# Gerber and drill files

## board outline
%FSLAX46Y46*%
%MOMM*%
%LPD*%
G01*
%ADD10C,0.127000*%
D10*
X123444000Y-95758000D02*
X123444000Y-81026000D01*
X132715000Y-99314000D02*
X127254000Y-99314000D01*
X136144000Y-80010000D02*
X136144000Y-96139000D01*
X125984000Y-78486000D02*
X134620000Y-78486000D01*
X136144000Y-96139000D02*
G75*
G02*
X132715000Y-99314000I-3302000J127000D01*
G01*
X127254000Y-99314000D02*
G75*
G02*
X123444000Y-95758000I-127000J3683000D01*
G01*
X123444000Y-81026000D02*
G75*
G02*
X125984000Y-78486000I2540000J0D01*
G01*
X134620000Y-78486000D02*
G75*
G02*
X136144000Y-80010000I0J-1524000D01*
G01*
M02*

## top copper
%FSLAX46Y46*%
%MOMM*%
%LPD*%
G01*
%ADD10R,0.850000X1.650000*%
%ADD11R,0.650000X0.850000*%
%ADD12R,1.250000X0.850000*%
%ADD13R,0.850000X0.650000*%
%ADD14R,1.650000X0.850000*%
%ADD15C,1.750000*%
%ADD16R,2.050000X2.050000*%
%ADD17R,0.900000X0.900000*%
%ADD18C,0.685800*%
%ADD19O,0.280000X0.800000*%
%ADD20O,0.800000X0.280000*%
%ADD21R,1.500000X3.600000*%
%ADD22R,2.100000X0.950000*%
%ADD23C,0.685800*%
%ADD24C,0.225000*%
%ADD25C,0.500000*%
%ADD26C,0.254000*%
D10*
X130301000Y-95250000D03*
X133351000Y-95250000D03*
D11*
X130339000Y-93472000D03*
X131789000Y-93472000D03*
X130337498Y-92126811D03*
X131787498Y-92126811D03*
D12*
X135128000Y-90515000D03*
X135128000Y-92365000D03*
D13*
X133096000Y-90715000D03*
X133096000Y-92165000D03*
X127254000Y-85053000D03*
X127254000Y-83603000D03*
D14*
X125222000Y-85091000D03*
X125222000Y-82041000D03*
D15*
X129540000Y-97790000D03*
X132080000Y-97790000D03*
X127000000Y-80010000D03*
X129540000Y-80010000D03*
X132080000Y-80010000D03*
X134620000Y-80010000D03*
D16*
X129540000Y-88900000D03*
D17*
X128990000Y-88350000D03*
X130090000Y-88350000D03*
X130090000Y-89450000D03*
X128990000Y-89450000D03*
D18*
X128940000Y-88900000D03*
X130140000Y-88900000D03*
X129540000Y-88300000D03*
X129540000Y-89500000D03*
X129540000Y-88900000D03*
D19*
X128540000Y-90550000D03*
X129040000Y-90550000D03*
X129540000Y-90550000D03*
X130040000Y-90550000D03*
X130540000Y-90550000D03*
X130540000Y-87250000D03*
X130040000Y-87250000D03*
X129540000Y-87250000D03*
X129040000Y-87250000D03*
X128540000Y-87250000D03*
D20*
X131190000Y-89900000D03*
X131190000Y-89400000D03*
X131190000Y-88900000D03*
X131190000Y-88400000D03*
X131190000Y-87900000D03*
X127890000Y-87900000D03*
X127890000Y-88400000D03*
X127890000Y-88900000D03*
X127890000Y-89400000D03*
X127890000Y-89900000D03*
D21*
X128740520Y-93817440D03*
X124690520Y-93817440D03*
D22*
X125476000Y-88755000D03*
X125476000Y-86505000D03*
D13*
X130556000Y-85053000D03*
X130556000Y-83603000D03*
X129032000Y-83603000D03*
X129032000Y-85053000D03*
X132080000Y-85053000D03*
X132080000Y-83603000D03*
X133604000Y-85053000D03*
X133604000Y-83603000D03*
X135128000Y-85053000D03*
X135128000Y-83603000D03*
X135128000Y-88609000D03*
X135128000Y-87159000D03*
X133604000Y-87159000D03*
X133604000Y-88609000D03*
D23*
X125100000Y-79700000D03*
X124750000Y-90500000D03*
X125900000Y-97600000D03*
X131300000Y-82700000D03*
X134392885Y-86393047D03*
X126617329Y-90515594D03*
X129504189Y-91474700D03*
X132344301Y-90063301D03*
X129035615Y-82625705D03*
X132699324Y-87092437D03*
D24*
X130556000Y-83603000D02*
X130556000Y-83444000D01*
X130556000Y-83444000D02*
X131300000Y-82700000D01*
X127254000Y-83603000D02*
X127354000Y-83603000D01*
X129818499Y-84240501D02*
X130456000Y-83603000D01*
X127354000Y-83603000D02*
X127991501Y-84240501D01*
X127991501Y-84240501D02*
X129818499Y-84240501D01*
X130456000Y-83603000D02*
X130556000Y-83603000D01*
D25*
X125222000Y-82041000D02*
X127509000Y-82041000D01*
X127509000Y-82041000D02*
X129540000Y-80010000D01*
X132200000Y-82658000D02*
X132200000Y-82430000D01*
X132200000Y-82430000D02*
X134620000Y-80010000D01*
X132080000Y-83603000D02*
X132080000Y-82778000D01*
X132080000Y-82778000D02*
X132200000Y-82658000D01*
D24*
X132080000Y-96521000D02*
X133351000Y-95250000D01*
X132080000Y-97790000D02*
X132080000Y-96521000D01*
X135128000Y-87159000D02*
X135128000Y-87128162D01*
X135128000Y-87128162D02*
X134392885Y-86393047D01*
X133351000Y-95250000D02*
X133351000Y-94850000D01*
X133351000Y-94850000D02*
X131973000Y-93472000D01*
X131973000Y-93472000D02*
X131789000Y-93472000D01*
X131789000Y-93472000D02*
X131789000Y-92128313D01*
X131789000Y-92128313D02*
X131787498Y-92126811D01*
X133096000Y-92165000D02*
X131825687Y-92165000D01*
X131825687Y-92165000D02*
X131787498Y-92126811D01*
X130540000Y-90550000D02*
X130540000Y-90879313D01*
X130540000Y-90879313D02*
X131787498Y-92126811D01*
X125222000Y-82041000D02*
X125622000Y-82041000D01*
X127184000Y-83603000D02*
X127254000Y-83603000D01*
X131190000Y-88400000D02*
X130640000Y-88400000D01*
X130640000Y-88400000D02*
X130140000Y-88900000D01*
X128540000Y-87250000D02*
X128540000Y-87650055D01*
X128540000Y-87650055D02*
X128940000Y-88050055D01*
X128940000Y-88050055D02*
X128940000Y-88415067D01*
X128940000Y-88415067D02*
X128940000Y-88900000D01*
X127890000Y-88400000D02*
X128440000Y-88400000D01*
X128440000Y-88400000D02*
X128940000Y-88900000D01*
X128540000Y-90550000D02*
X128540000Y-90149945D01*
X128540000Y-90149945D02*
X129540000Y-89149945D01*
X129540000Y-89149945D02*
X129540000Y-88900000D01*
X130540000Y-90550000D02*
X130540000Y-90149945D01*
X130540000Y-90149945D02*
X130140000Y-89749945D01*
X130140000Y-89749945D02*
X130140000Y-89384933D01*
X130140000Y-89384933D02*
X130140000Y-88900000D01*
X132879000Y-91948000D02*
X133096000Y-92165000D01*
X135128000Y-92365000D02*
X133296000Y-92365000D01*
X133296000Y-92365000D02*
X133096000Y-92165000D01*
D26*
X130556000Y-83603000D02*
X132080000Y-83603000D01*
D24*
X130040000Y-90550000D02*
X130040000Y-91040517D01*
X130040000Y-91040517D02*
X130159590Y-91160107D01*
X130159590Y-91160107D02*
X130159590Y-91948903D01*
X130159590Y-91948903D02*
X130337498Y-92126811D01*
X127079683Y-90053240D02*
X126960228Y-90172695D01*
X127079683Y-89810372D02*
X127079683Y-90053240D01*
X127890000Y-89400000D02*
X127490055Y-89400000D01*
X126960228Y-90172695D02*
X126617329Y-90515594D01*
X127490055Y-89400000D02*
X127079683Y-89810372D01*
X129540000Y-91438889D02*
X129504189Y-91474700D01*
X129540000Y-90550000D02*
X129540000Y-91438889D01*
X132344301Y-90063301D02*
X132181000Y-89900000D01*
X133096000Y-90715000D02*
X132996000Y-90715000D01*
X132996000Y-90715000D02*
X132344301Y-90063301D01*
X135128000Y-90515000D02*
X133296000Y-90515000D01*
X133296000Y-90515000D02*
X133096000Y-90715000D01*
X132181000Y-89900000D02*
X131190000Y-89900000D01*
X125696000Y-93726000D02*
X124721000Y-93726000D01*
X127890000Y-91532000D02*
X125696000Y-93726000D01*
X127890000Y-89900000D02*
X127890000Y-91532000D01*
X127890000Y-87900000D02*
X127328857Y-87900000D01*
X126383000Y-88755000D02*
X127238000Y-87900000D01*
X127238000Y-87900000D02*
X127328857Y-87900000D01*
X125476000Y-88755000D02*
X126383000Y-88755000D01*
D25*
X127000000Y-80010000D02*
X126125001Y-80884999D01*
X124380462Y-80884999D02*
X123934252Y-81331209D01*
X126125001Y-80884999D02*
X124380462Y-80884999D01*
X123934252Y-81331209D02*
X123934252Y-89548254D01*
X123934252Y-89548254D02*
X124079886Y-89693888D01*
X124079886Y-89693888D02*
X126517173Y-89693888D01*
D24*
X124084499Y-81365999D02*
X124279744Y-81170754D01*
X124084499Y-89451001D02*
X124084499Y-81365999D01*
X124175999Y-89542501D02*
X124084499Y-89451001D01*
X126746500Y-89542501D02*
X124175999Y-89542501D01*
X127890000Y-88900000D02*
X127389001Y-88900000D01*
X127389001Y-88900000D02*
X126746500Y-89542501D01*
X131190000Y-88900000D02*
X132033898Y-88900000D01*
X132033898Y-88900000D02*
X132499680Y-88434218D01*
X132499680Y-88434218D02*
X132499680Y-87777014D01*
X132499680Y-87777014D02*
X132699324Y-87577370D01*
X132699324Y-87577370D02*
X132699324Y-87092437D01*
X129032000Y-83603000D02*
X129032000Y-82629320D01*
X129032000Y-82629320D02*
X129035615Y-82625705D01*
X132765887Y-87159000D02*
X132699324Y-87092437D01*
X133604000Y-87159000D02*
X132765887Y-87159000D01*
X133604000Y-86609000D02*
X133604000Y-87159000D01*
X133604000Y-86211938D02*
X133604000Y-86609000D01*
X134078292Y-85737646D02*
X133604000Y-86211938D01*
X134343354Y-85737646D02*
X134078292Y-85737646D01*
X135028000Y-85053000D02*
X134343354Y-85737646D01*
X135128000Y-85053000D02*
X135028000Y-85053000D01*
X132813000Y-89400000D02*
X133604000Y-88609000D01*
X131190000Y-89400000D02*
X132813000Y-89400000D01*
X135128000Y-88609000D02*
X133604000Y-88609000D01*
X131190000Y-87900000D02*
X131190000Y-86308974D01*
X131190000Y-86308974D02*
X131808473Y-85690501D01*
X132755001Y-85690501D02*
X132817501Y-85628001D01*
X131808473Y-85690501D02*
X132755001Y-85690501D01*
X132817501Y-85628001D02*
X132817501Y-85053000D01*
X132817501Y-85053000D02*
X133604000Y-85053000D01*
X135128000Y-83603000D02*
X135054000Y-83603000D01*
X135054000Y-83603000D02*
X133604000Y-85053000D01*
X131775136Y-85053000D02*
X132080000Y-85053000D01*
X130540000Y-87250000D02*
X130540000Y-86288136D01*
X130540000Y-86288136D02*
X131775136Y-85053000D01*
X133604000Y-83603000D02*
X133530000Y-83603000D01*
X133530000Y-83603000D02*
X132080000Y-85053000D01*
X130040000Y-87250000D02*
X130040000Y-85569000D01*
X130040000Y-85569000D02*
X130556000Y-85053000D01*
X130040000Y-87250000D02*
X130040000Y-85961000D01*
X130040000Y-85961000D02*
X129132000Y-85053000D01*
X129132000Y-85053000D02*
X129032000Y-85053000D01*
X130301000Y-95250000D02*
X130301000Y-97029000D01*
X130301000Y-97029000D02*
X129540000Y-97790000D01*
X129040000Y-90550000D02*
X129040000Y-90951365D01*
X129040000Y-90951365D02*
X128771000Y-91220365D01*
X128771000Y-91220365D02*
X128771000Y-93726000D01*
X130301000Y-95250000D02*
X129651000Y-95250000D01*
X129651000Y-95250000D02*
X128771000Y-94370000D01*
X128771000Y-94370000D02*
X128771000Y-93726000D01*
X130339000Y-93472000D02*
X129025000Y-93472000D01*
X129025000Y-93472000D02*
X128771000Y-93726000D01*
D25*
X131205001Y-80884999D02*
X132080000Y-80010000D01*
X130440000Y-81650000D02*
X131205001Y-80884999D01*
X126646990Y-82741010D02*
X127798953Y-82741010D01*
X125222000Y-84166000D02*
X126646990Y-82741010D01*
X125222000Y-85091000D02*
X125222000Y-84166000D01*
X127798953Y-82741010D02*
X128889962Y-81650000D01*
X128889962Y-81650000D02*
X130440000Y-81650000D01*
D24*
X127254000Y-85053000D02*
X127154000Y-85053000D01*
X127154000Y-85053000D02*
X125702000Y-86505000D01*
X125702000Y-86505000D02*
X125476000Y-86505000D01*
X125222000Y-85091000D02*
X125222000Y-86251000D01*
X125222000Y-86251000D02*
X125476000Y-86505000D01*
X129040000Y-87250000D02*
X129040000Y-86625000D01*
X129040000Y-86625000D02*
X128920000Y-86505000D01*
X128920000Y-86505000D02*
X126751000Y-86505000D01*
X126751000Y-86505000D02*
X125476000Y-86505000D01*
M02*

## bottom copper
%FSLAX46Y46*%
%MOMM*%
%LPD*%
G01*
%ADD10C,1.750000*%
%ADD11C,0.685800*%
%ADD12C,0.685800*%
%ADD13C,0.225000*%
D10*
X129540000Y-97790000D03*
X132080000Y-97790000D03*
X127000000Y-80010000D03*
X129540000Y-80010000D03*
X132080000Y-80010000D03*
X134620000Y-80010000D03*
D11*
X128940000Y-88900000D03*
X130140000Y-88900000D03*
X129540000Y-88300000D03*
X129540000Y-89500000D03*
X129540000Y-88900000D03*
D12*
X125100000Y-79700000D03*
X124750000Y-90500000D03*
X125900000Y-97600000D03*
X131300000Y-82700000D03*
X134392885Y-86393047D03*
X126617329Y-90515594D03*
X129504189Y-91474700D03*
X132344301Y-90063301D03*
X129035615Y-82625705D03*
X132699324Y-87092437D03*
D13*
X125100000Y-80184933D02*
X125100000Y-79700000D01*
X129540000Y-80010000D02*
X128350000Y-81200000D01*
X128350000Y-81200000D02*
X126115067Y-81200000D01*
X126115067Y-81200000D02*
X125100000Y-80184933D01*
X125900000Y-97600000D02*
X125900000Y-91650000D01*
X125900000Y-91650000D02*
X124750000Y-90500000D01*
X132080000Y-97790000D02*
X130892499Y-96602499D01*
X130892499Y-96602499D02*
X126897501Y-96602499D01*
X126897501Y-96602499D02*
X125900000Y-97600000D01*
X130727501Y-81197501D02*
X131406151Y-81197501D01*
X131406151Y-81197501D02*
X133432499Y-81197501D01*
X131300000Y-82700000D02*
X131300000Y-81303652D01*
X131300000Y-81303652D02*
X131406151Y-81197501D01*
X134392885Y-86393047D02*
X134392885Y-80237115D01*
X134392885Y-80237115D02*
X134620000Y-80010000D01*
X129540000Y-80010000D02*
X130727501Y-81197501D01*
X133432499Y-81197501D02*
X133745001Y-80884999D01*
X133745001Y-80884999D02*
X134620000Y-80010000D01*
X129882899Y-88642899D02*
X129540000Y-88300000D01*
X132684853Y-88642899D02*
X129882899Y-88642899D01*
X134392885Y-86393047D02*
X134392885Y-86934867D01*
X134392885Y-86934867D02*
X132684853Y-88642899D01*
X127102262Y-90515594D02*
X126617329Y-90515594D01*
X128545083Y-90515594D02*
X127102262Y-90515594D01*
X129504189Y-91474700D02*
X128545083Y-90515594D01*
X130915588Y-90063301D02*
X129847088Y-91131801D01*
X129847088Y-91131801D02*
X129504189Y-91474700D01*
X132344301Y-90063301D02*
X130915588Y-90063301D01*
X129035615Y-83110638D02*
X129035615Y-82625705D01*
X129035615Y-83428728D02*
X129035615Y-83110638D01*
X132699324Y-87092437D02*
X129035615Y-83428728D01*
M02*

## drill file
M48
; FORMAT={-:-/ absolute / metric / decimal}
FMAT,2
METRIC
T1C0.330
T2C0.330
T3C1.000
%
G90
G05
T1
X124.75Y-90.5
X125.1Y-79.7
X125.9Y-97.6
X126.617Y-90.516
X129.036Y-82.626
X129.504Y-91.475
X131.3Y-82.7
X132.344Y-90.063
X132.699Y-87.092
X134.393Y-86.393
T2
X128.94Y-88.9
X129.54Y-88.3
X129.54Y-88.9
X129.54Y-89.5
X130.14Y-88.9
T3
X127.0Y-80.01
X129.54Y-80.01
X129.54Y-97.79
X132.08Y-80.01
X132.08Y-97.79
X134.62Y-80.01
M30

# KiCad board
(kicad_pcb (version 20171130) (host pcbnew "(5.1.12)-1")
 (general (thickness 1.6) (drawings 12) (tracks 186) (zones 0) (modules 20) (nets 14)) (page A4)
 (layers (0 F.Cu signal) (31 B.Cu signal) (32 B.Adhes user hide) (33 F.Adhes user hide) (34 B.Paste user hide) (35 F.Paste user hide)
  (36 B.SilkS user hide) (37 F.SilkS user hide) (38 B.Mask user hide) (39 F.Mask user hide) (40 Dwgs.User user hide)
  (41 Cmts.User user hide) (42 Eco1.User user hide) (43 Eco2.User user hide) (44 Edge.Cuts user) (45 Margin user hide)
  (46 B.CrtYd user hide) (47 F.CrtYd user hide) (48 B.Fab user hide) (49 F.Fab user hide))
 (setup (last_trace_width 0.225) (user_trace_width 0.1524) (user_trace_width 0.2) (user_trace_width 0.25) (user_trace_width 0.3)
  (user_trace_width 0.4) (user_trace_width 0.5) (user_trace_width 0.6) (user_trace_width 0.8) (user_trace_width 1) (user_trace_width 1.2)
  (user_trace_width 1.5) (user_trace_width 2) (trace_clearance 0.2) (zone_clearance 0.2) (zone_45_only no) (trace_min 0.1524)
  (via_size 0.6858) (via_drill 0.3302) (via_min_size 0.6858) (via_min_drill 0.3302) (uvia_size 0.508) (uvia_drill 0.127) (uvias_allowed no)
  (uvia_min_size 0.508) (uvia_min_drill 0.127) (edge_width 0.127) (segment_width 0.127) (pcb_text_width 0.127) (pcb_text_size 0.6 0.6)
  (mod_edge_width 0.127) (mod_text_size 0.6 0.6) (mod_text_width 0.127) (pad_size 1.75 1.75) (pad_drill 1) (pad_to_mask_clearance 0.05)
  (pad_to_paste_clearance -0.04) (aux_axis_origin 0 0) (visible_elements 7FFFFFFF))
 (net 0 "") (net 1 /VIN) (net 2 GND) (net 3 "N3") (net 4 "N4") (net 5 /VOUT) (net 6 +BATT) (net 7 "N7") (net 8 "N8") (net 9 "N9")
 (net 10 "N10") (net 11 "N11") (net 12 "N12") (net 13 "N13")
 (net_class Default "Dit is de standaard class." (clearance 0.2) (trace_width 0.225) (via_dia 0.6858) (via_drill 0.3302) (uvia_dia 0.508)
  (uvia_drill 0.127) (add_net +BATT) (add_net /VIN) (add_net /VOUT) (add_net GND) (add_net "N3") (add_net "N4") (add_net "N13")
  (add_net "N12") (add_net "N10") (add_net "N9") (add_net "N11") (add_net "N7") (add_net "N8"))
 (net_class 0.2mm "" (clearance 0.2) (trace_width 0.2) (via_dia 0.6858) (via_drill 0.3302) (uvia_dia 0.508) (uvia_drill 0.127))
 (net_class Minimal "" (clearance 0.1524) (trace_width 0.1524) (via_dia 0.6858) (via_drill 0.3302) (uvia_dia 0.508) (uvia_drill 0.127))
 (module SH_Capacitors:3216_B (layer F.Cu) (at 131.826 95.25) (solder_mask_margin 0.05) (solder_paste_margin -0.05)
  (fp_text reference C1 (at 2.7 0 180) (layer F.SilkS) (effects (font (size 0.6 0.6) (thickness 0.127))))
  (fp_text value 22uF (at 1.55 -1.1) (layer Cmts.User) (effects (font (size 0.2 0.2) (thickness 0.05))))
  (pad 1 smd rect (at -1.525 0) (size 0.85 1.65) (layers F.Cu F.Paste F.Mask) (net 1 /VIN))
  (pad 2 smd rect (at 1.525 0) (size 0.85 1.65) (layers F.Cu F.Paste F.Mask) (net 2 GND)))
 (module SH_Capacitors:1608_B (layer F.Cu) (at 131.064 93.472) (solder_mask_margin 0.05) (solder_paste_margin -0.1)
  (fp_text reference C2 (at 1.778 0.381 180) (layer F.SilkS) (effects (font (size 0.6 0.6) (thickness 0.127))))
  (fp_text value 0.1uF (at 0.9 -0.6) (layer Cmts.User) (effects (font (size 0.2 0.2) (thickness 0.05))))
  (pad 1 smd rect (at -0.725 0) (size 0.65 0.85) (layers F.Cu F.Paste F.Mask) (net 1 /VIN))
  (pad 2 smd rect (at 0.725 0) (size 0.65 0.85) (layers F.Cu F.Paste F.Mask) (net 2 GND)))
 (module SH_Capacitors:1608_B (layer F.Cu) (at 131.062498 92.126811) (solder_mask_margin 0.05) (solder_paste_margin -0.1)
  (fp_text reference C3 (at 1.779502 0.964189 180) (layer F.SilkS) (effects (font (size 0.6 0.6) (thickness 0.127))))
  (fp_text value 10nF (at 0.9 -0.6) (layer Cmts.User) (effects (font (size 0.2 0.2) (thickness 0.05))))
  (pad 1 smd rect (at -0.725 0) (size 0.65 0.85) (layers F.Cu F.Paste F.Mask) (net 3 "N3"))
  (pad 2 smd rect (at 0.725 0) (size 0.65 0.85) (layers F.Cu F.Paste F.Mask) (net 2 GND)))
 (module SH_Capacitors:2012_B (layer F.Cu) (at 135.128 91.44 270) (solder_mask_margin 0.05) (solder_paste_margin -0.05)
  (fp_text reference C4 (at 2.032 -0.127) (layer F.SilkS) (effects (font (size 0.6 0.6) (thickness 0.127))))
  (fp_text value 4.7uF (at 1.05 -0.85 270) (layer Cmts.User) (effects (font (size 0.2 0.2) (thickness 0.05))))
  (pad 1 smd rect (at -0.925 0 270) (size 0.85 1.25) (layers F.Cu F.Paste F.Mask) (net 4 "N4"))
  (pad 2 smd rect (at 0.925 0 270) (size 0.85 1.25) (layers F.Cu F.Paste F.Mask) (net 2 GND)))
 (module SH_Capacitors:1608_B (layer F.Cu) (at 133.096 91.44 270) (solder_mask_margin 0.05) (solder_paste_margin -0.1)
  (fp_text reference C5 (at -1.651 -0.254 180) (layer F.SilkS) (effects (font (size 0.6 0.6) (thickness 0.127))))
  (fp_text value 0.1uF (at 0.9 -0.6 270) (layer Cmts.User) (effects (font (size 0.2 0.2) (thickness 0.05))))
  (pad 1 smd rect (at -0.725 0 270) (size 0.65 0.85) (layers F.Cu F.Paste F.Mask) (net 4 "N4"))
  (pad 2 smd rect (at 0.725 0 270) (size 0.65 0.85) (layers F.Cu F.Paste F.Mask) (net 2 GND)))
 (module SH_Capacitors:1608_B (layer F.Cu) (at 127.254 84.328 90) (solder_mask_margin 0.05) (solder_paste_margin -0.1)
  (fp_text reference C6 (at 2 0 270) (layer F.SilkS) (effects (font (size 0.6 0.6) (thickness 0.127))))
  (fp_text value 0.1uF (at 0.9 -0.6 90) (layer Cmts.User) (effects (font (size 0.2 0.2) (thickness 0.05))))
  (pad 1 smd rect (at -0.725 0 90) (size 0.65 0.85) (layers F.Cu F.Paste F.Mask) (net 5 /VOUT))
  (pad 2 smd rect (at 0.725 0 90) (size 0.65 0.85) (layers F.Cu F.Paste F.Mask) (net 2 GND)))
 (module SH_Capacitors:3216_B (layer F.Cu) (at 125.222 83.566 90) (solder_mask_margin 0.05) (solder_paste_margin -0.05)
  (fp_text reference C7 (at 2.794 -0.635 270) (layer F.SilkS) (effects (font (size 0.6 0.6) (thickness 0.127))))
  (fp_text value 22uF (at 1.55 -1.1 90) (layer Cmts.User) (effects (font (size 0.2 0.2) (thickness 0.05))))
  (pad 1 smd rect (at -1.525 0 90) (size 0.85 1.65) (layers F.Cu F.Paste F.Mask) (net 5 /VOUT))
  (pad 2 smd rect (at 1.525 0 90) (size 0.85 1.65) (layers F.Cu F.Paste F.Mask) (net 2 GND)))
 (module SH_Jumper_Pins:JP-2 (layer F.Cu) (at 130.81 97.79)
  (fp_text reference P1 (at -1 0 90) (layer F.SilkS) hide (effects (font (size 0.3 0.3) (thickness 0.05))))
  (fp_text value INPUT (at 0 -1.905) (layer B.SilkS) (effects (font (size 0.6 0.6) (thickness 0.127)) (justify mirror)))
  (pad 1 thru_hole circle (at -1.27 0) (size 1.75 1.75) (drill 1) (layers *.Cu *.Mask) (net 1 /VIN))
  (pad 2 thru_hole circle (at 1.27 0) (size 1.75 1.75) (drill 1) (layers *.Cu *.Mask) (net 2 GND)))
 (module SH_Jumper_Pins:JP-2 (layer F.Cu) (at 128.27 80.01)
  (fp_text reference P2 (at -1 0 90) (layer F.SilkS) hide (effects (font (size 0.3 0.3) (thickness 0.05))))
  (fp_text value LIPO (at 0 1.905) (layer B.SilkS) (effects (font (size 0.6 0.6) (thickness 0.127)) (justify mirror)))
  (pad 1 thru_hole circle (at -1.27 0) (size 1.75 1.75) (drill 1) (layers *.Cu *.Mask) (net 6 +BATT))
  (pad 2 thru_hole circle (at 1.27 0) (size 1.75 1.75) (drill 1) (layers *.Cu *.Mask) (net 2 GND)))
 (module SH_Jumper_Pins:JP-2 (layer F.Cu) (at 133.35 80.01)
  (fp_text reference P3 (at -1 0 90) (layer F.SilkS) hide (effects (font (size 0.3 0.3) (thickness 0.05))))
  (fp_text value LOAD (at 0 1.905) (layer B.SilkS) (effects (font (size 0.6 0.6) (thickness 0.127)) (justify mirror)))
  (pad 1 thru_hole circle (at -1.27 0) (size 1.75 1.75) (drill 1) (layers *.Cu *.Mask) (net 5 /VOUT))
  (pad 2 thru_hole circle (at 1.27 0) (size 1.75 1.75) (drill 1) (layers *.Cu *.Mask) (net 2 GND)))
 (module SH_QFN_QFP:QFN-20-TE (layer F.Cu) (at 129.54 88.9) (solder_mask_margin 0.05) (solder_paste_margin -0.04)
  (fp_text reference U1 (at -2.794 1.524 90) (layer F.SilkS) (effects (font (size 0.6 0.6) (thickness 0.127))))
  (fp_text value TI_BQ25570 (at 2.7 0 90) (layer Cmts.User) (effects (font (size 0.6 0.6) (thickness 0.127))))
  (pad 21 smd rect (at 0 0) (size 2.05 2.05) (layers F.Cu F.Mask) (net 2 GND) (zone_connect 2))
  (pad 21 smd rect (at -0.55 -0.55) (size 0.9 0.9) (layers F.Cu F.Paste F.Mask) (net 2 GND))
  (pad 21 smd rect (at 0.55 -0.55) (size 0.9 0.9) (layers F.Cu F.Paste F.Mask) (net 2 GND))
  (pad 21 smd rect (at 0.55 0.55) (size 0.9 0.9) (layers F.Cu F.Paste F.Mask) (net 2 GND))
  (pad 21 smd rect (at -0.55 0.55) (size 0.9 0.9) (layers F.Cu F.Paste F.Mask) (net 2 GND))
  (pad 21 thru_hole circle (at -0.6 0) (size 0.6858 0.6858) (drill 0.3302) (layers *.Cu) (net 2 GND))
  (pad 21 thru_hole circle (at 0.6 0) (size 0.6858 0.6858) (drill 0.3302) (layers *.Cu) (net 2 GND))
  (pad 21 thru_hole circle (at 0 -0.6) (size 0.6858 0.6858) (drill 0.3302) (layers *.Cu) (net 2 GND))
  (pad 21 thru_hole circle (at 0 0.6) (size 0.6858 0.6858) (drill 0.3302) (layers *.Cu) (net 2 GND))
  (pad 21 thru_hole circle (at 0 0) (size 0.6858 0.6858) (drill 0.3302) (layers *.Cu) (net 2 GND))
  (pad 1 smd oval (at -1 1.65) (size 0.28 0.8) (layers F.Cu F.Paste F.Mask) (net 2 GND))
  (pad 2 smd oval (at -0.5 1.65) (size 0.28 0.8) (layers F.Cu F.Paste F.Mask) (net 1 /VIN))
  (pad 3 smd oval (at 0 1.65) (size 0.28 0.8) (layers F.Cu F.Paste F.Mask) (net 4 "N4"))
  (pad 4 smd oval (at 0.5 1.65) (size 0.28 0.8) (layers F.Cu F.Paste F.Mask) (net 3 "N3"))
  (pad 5 smd oval (at 1 1.65) (size 0.28 0.8) (layers F.Cu F.Paste F.Mask) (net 2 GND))
  (pad 11 smd oval (at 1 -1.65) (size 0.28 0.8) (layers F.Cu F.Paste F.Mask) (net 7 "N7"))
  (pad 12 smd oval (at 0.5 -1.65) (size 0.28 0.8) (layers F.Cu F.Paste F.Mask) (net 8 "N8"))
  (pad 13 smd oval (at 0 -1.65) (size 0.28 0.8) (layers F.Cu F.Paste F.Mask))
  (pad 14 smd oval (at -0.5 -1.65) (size 0.28 0.8) (layers F.Cu F.Paste F.Mask) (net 5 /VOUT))
  (pad 15 smd oval (at -1 -1.65) (size 0.28 0.8) (layers F.Cu F.Paste F.Mask) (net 2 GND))
  (pad 6 smd oval (at 1.65 1 90) (size 0.28 0.8) (layers F.Cu F.Paste F.Mask) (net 4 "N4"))
  (pad 7 smd oval (at 1.65 0.5 90) (size 0.28 0.8) (layers F.Cu F.Paste F.Mask) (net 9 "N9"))
  (pad 8 smd oval (at 1.65 0 90) (size 0.28 0.8) (layers F.Cu F.Paste F.Mask) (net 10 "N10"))
  (pad 9 smd oval (at 1.65 -0.5 90) (size 0.28 0.8) (layers F.Cu F.Paste F.Mask) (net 2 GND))
  (pad 10 smd oval (at 1.65 -1 90) (size 0.28 0.8) (layers F.Cu F.Paste F.Mask) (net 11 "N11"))
  (pad 16 smd oval (at -1.65 -1 90) (size 0.28 0.8) (layers F.Cu F.Paste F.Mask) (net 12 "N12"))
  (pad 17 smd oval (at -1.65 -0.5 90) (size 0.28 0.8) (layers F.Cu F.Paste F.Mask) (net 2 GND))
  (pad 18 smd oval (at -1.65 0 90) (size 0.28 0.8) (layers F.Cu F.Paste F.Mask) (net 6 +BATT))
  (pad 19 smd oval (at -1.65 0.5 90) (size 0.28 0.8) (layers F.Cu F.Paste F.Mask) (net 4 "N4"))
  (pad 20 smd oval (at -1.65 1 90) (size 0.28 0.8) (layers F.Cu F.Paste F.Mask) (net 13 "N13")))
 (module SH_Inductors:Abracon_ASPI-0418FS (layer F.Cu) (at 126.71552 93.81744 180) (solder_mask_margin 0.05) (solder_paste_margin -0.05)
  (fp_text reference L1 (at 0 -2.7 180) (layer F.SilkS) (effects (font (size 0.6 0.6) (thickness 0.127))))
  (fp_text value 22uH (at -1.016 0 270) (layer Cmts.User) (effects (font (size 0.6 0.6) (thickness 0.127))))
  (pad 1 smd rect (at -2.025 0 180) (size 1.5 3.6) (layers F.Cu F.Paste F.Mask) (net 1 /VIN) (zone_connect 2))
  (pad 2 smd rect (at 2.025 0 180) (size 1.5 3.6) (layers F.Cu F.Paste F.Mask) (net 13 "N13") (zone_connect 2)))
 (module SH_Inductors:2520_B (layer F.Cu) (at 125.476 87.63 90) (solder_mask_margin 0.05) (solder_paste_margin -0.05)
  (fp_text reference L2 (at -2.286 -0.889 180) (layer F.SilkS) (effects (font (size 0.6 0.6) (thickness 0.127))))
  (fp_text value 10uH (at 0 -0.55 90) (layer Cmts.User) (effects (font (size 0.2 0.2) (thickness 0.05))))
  (pad 1 smd rect (at -1.125 0 90) (size 0.95 2.1) (layers F.Cu F.Paste F.Mask) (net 12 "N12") (zone_connect 2))
  (pad 2 smd rect (at 1.125 0 90) (size 0.95 2.1) (layers F.Cu F.Paste F.Mask) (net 5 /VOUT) (zone_connect 2)))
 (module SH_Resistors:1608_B (layer F.Cu) (at 130.556 84.328 90) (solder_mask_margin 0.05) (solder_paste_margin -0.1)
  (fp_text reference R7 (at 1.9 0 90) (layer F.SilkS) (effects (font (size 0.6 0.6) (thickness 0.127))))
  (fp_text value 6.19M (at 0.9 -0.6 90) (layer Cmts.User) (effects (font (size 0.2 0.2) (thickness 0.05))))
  (pad 1 smd rect (at -0.725 0 90) (size 0.65 0.85) (layers F.Cu F.Paste F.Mask) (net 8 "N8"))
  (pad 2 smd rect (at 0.725 0 90) (size 0.65 0.85) (layers F.Cu F.Paste F.Mask) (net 2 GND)))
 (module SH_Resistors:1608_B (layer F.Cu) (at 129.032 84.328 270) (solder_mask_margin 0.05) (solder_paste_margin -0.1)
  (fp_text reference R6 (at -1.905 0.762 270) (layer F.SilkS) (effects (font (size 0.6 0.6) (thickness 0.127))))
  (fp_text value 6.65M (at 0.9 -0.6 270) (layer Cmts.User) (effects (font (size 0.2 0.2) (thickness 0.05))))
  (pad 1 smd rect (at -0.725 0 270) (size 0.65 0.85) (layers F.Cu F.Paste F.Mask) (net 10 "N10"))
  (pad 2 smd rect (at 0.725 0 270) (size 0.65 0.85) (layers F.Cu F.Paste F.Mask) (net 8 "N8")))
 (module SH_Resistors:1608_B (layer F.Cu) (at 132.08 84.328 90) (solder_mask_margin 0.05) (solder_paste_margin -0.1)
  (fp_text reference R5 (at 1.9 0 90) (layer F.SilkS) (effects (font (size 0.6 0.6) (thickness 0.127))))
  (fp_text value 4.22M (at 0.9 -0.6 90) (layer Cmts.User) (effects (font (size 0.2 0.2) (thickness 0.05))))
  (pad 1 smd rect (at -0.725 0 90) (size 0.65 0.85) (layers F.Cu F.Paste F.Mask) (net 7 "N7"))
  (pad 2 smd rect (at 0.725 0 90) (size 0.65 0.85) (layers F.Cu F.Paste F.Mask) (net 2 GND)))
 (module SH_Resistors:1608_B (layer F.Cu) (at 133.604 84.328 90) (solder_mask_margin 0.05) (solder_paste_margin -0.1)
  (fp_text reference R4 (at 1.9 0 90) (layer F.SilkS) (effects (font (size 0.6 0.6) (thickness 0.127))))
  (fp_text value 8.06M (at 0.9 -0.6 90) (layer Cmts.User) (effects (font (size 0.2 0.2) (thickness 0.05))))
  (pad 1 smd rect (at -0.725 0 90) (size 0.65 0.85) (layers F.Cu F.Paste F.Mask) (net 11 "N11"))
  (pad 2 smd rect (at 0.725 0 90) (size 0.65 0.85) (layers F.Cu F.Paste F.Mask) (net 7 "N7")))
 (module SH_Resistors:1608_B (layer F.Cu) (at 135.128 84.328 90) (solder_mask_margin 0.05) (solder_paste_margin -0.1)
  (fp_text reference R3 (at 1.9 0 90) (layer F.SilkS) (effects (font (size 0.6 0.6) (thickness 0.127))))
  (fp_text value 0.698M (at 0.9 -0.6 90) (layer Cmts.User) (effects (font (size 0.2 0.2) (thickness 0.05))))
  (pad 1 smd rect (at -0.725 0 90) (size 0.65 0.85) (layers F.Cu F.Paste F.Mask) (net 10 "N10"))
  (pad 2 smd rect (at 0.725 0 90) (size 0.65 0.85) (layers F.Cu F.Paste F.Mask) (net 11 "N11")))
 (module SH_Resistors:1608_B (layer F.Cu) (at 135.128 87.884 90) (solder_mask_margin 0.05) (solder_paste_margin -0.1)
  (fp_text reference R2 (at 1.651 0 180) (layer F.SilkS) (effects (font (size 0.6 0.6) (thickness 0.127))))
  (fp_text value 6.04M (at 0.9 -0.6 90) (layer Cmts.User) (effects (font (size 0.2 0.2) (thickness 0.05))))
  (pad 1 smd rect (at -0.725 0 90) (size 0.65 0.85) (layers F.Cu F.Paste F.Mask) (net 9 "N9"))
  (pad 2 smd rect (at 0.725 0 90) (size 0.65 0.85) (layers F.Cu F.Paste F.Mask) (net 2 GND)))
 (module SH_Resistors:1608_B (layer F.Cu) (at 133.604 87.884 270) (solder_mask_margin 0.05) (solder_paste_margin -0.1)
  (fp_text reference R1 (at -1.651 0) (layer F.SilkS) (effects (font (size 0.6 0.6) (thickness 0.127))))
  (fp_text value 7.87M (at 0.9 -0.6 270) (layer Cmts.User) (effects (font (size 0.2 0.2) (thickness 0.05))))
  (pad 1 smd rect (at -0.725 0 270) (size 0.65 0.85) (layers F.Cu F.Paste F.Mask) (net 10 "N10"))
  (pad 2 smd rect (at 0.725 0 270) (size 0.65 0.85) (layers F.Cu F.Paste F.Mask) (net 9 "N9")))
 (gr_line (start 123.444 95.758) (end 123.444 81.026) (angle 90) (layer Edge.Cuts) (width 0.127))
 (gr_line (start 132.715 99.314) (end 127.254 99.314) (angle 90) (layer Edge.Cuts) (width 0.127))
 (gr_line (start 136.144 80.01) (end 136.144 96.139) (angle 90) (layer Edge.Cuts) (width 0.127))
 (gr_line (start 125.984 78.486) (end 134.62 78.486) (angle 90) (layer Edge.Cuts) (width 0.127))
 (gr_arc (start 132.842 96.012) (end 136.144 96.139) (angle 90) (layer Edge.Cuts) (width 0.127))
 (gr_arc (start 127.127 95.631) (end 127.254 99.314) (angle 90) (layer Edge.Cuts) (width 0.127))
 (gr_arc (start 125.984 81.026) (end 123.444 81.026) (angle 90) (layer Edge.Cuts) (width 0.127))
 (gr_arc (start 134.62 80.01) (end 134.62 78.486) (angle 90) (layer Edge.Cuts) (width 0.127))
 (segment (start 125.1 80.184933) (end 125.1 79.7) (width 0.225) (layer B.Cu) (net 2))
 (segment (start 129.54 80.01) (end 128.35 81.2) (width 0.225) (layer B.Cu) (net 2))
 (segment (start 128.35 81.2) (end 126.115067 81.2) (width 0.225) (layer B.Cu) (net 2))
 (segment (start 126.115067 81.2) (end 125.1 80.184933) (width 0.225) (layer B.Cu) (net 2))
 (segment (start 125.9 97.6) (end 125.9 91.65) (width 0.225) (layer B.Cu) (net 2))
 (segment (start 125.9 91.65) (end 124.75 90.5) (width 0.225) (layer B.Cu) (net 2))
 (segment (start 132.08 97.79) (end 130.892499 96.602499) (width 0.225) (layer B.Cu) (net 2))
 (segment (start 130.892499 96.602499) (end 126.897501 96.602499) (width 0.225) (layer B.Cu) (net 2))
 (segment (start 126.897501 96.602499) (end 125.9 97.6) (width 0.225) (layer B.Cu) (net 2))
 (segment (start 130.727501 81.197501) (end 131.406151 81.197501) (width 0.225) (layer B.Cu) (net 2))
 (segment (start 131.406151 81.197501) (end 133.432499 81.197501) (width 0.225) (layer B.Cu) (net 2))
 (segment (start 131.3 82.7) (end 131.3 81.303652) (width 0.225) (layer B.Cu) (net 2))
 (segment (start 131.3 81.303652) (end 131.406151 81.197501) (width 0.225) (layer B.Cu) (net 2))
 (segment (start 130.556 83.603) (end 130.556 83.444) (width 0.225) (layer F.Cu) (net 2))
 (segment (start 130.556 83.444) (end 131.3 82.7) (width 0.225) (layer F.Cu) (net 2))
 (segment (start 134.392885 86.393047) (end 134.392885 80.237115) (width 0.225) (layer B.Cu) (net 2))
 (segment (start 134.392885 80.237115) (end 134.62 80.01) (width 0.225) (layer B.Cu) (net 2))
 (segment (start 129.54 80.01) (end 130.727501 81.197501) (width 0.225) (layer B.Cu) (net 2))
 (segment (start 133.432499 81.197501) (end 133.745001 80.884999) (width 0.225) (layer B.Cu) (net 2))
 (segment (start 133.745001 80.884999) (end 134.62 80.01) (width 0.225) (layer B.Cu) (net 2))
 (segment (start 127.254 83.603) (end 127.354 83.603) (width 0.225) (layer F.Cu) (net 2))
 (segment (start 129.818499 84.240501) (end 130.456 83.603) (width 0.225) (layer F.Cu) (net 2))
 (segment (start 127.354 83.603) (end 127.991501 84.240501) (width 0.225) (layer F.Cu) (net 2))
 (segment (start 127.991501 84.240501) (end 129.818499 84.240501) (width 0.225) (layer F.Cu) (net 2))
 (segment (start 130.456 83.603) (end 130.556 83.603) (width 0.225) (layer F.Cu) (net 2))
 (segment (start 125.222 82.041) (end 127.509 82.041) (width 0.5) (layer F.Cu) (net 2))
 (segment (start 127.509 82.041) (end 129.54 80.01) (width 0.5) (layer F.Cu) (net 2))
 (segment (start 132.2 82.658) (end 132.2 82.43) (width 0.5) (layer F.Cu) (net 2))
 (segment (start 132.2 82.43) (end 134.62 80.01) (width 0.5) (layer F.Cu) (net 2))
 (segment (start 132.08 83.603) (end 132.08 82.778) (width 0.5) (layer F.Cu) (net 2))
 (segment (start 132.08 82.778) (end 132.2 82.658) (width 0.5) (layer F.Cu) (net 2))
 (segment (start 132.08 96.521) (end 133.351 95.25) (width 0.225) (layer F.Cu) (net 2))
 (segment (start 132.08 97.79) (end 132.08 96.521) (width 0.225) (layer F.Cu) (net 2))
 (segment (start 129.882899 88.642899) (end 129.54 88.3) (width 0.225) (layer B.Cu) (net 2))
 (segment (start 132.684853 88.642899) (end 129.882899 88.642899) (width 0.225) (layer B.Cu) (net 2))
 (segment (start 134.392885 86.393047) (end 134.392885 86.934867) (width 0.225) (layer B.Cu) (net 2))
 (segment (start 134.392885 86.934867) (end 132.684853 88.642899) (width 0.225) (layer B.Cu) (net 2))
 (segment (start 135.128 87.159) (end 135.128 87.128162) (width 0.225) (layer F.Cu) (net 2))
 (segment (start 135.128 87.128162) (end 134.392885 86.393047) (width 0.225) (layer F.Cu) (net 2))
 (segment (start 133.351 95.25) (end 133.351 94.85) (width 0.225) (layer F.Cu) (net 2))
 (segment (start 133.351 94.85) (end 131.973 93.472) (width 0.225) (layer F.Cu) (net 2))
 (segment (start 131.973 93.472) (end 131.789 93.472) (width 0.225) (layer F.Cu) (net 2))
 (segment (start 131.789 93.472) (end 131.789 92.128313) (width 0.225) (layer F.Cu) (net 2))
 (segment (start 131.789 92.128313) (end 131.787498 92.126811) (width 0.225) (layer F.Cu) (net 2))
 (segment (start 133.096 92.165) (end 131.825687 92.165) (width 0.225) (layer F.Cu) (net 2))
 (segment (start 131.825687 92.165) (end 131.787498 92.126811) (width 0.225) (layer F.Cu) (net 2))
 (segment (start 130.54 90.55) (end 130.54 90.879313) (width 0.225) (layer F.Cu) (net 2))
 (segment (start 130.54 90.879313) (end 131.787498 92.126811) (width 0.225) (layer F.Cu) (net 2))
 (segment (start 125.222 82.041) (end 125.622 82.041) (width 0.225) (layer F.Cu) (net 2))
 (segment (start 127.184 83.603) (end 127.254 83.603) (width 0.225) (layer F.Cu) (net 2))
 (segment (start 131.19 88.4) (end 130.64 88.4) (width 0.225) (layer F.Cu) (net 2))
 (segment (start 130.64 88.4) (end 130.14 88.9) (width 0.225) (layer F.Cu) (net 2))
 (segment (start 128.54 87.25) (end 128.54 87.650055) (width 0.225) (layer F.Cu) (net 2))
 (segment (start 128.54 87.650055) (end 128.94 88.050055) (width 0.225) (layer F.Cu) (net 2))
 (segment (start 128.94 88.050055) (end 128.94 88.415067) (width 0.225) (layer F.Cu) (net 2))
 (segment (start 128.94 88.415067) (end 128.94 88.9) (width 0.225) (layer F.Cu) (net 2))
 (segment (start 127.89 88.4) (end 128.44 88.4) (width 0.225) (layer F.Cu) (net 2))
 (segment (start 128.44 88.4) (end 128.94 88.9) (width 0.225) (layer F.Cu) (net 2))
 (segment (start 128.54 90.55) (end 128.54 90.149945) (width 0.225) (layer F.Cu) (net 2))
 (segment (start 128.54 90.149945) (end 129.54 89.149945) (width 0.225) (layer F.Cu) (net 2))
 (segment (start 129.54 89.149945) (end 129.54 88.9) (width 0.225) (layer F.Cu) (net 2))
 (segment (start 130.54 90.55) (end 130.54 90.149945) (width 0.225) (layer F.Cu) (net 2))
 (segment (start 130.54 90.149945) (end 130.14 89.749945) (width 0.225) (layer F.Cu) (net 2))
 (segment (start 130.14 89.749945) (end 130.14 89.384933) (width 0.225) (layer F.Cu) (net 2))
 (segment (start 130.14 89.384933) (end 130.14 88.9) (width 0.225) (layer F.Cu) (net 2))
 (segment (start 132.879 91.948) (end 133.096 92.165) (width 0.225) (layer F.Cu) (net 2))
 (segment (start 135.128 92.365) (end 133.296 92.365) (width 0.225) (layer F.Cu) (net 2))
 (segment (start 133.296 92.365) (end 133.096 92.165) (width 0.225) (layer F.Cu) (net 2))
 (segment (start 130.556 83.603) (end 132.08 83.603) (width 0.254) (layer F.Cu) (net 2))
 (segment (start 130.04 90.55) (end 130.04 91.040517) (width 0.225) (layer F.Cu) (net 3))
 (segment (start 130.04 91.040517) (end 130.15959 91.160107) (width 0.225) (layer F.Cu) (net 3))
 (segment (start 130.15959 91.160107) (end 130.15959 91.948903) (width 0.225) (layer F.Cu) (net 3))
 (segment (start 130.15959 91.948903) (end 130.337498 92.126811) (width 0.225) (layer F.Cu) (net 3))
 (segment (start 127.079683 90.05324) (end 126.960228 90.172695) (width 0.225) (layer F.Cu) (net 4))
 (segment (start 127.079683 89.810372) (end 127.079683 90.05324) (width 0.225) (layer F.Cu) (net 4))
 (segment (start 127.89 89.4) (end 127.490055 89.4) (width 0.225) (layer F.Cu) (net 4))
 (segment (start 127.102262 90.515594) (end 126.617329 90.515594) (width 0.225) (layer B.Cu) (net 4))
 (segment (start 128.545083 90.515594) (end 127.102262 90.515594) (width 0.225) (layer B.Cu) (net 4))
 (segment (start 126.960228 90.172695) (end 126.617329 90.515594) (width 0.225) (layer F.Cu) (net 4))
 (segment (start 129.504189 91.4747) (end 128.545083 90.515594) (width 0.225) (layer B.Cu) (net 4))
 (segment (start 127.490055 89.4) (end 127.079683 89.810372) (width 0.225) (layer F.Cu) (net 4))
 (segment (start 130.915588 90.063301) (end 129.847088 91.131801) (width 0.225) (layer B.Cu) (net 4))
 (segment (start 129.847088 91.131801) (end 129.504189 91.4747) (width 0.225) (layer B.Cu) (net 4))
 (segment (start 132.344301 90.063301) (end 130.915588 90.063301) (width 0.225) (layer B.Cu) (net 4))
 (segment (start 129.54 91.438889) (end 129.504189 91.4747) (width 0.225) (layer F.Cu) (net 4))
 (segment (start 129.54 90.55) (end 129.54 91.438889) (width 0.225) (layer F.Cu) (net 4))
 (segment (start 132.344301 90.063301) (end 132.181 89.9) (width 0.225) (layer F.Cu) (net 4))
 (segment (start 133.096 90.715) (end 132.996 90.715) (width 0.225) (layer F.Cu) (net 4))
 (segment (start 132.996 90.715) (end 132.344301 90.063301) (width 0.225) (layer F.Cu) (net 4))
 (segment (start 135.128 90.515) (end 133.296 90.515) (width 0.225) (layer F.Cu) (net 4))
 (segment (start 133.296 90.515) (end 133.096 90.715) (width 0.225) (layer F.Cu) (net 4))
 (segment (start 132.181 89.9) (end 131.19 89.9) (width 0.225) (layer F.Cu) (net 4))
 (segment (start 125.696 93.726) (end 124.721 93.726) (width 0.225) (layer F.Cu) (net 13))
 (segment (start 127.89 91.532) (end 125.696 93.726) (width 0.225) (layer F.Cu) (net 13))
 (segment (start 127.89 89.9) (end 127.89 91.532) (width 0.225) (layer F.Cu) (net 13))
 (segment (start 127.89 87.9) (end 127.328857 87.9) (width 0.225) (layer F.Cu) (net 12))
 (segment (start 126.383 88.755) (end 127.238 87.9) (width 0.225) (layer F.Cu) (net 12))
 (segment (start 127.238 87.9) (end 127.328857 87.9) (width 0.225) (layer F.Cu) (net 12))
 (segment (start 125.476 88.755) (end 126.383 88.755) (width 0.225) (layer F.Cu) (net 12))
 (segment (start 127 80.01) (end 126.125001 80.884999) (width 0.5) (layer F.Cu) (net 6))
 (segment (start 124.380462 80.884999) (end 123.934252 81.331209) (width 0.5) (layer F.Cu) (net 6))
 (segment (start 126.125001 80.884999) (end 124.380462 80.884999) (width 0.5) (layer F.Cu) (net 6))
 (segment (start 123.934252 81.331209) (end 123.934252 89.548254) (width 0.5) (layer F.Cu) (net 6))
 (segment (start 123.934252 89.548254) (end 124.079886 89.693888) (width 0.5) (layer F.Cu) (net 6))
 (segment (start 124.079886 89.693888) (end 126.517173 89.693888) (width 0.5) (layer F.Cu) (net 6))
 (segment (start 124.084499 81.365999) (end 124.279744 81.170754) (width 0.225) (layer F.Cu) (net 6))
 (segment (start 124.084499 89.451001) (end 124.084499 81.365999) (width 0.225) (layer F.Cu) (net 6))
 (segment (start 124.175999 89.542501) (end 124.084499 89.451001) (width 0.225) (layer F.Cu) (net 6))
 (segment (start 126.7465 89.542501) (end 124.175999 89.542501) (width 0.225) (layer F.Cu) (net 6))
 (segment (start 127.89 88.9) (end 127.389001 88.9) (width 0.225) (layer F.Cu) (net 6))
 (segment (start 127.389001 88.9) (end 126.7465 89.542501) (width 0.225) (layer F.Cu) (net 6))
 (segment (start 131.19 88.9) (end 132.033898 88.9) (width 0.225) (layer F.Cu) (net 10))
 (segment (start 132.033898 88.9) (end 132.49968 88.434218) (width 0.225) (layer F.Cu) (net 10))
 (segment (start 132.49968 88.434218) (end 132.49968 87.777014) (width 0.225) (layer F.Cu) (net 10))
 (segment (start 132.49968 87.777014) (end 132.699324 87.57737) (width 0.225) (layer F.Cu) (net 10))
 (segment (start 132.699324 87.57737) (end 132.699324 87.092437) (width 0.225) (layer F.Cu) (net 10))
 (segment (start 129.035615 83.110638) (end 129.035615 82.625705) (width 0.225) (layer B.Cu) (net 10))
 (segment (start 129.035615 83.428728) (end 129.035615 83.110638) (width 0.225) (layer B.Cu) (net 10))
 (segment (start 132.699324 87.092437) (end 129.035615 83.428728) (width 0.225) (layer B.Cu) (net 10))
 (segment (start 129.032 83.603) (end 129.032 82.62932) (width 0.225) (layer F.Cu) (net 10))
 (segment (start 129.032 82.62932) (end 129.035615 82.625705) (width 0.225) (layer F.Cu) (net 10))
 (segment (start 132.765887 87.159) (end 132.699324 87.092437) (width 0.225) (layer F.Cu) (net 10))
 (segment (start 133.604 87.159) (end 132.765887 87.159) (width 0.225) (layer F.Cu) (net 10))
 (segment (start 133.604 86.609) (end 133.604 87.159) (width 0.225) (layer F.Cu) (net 10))
 (segment (start 133.604 86.211938) (end 133.604 86.609) (width 0.225) (layer F.Cu) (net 10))
 (segment (start 134.078292 85.737646) (end 133.604 86.211938) (width 0.225) (layer F.Cu) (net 10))
 (segment (start 134.343354 85.737646) (end 134.078292 85.737646) (width 0.225) (layer F.Cu) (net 10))
 (segment (start 135.028 85.053) (end 134.343354 85.737646) (width 0.225) (layer F.Cu) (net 10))
 (segment (start 135.128 85.053) (end 135.028 85.053) (width 0.225) (layer F.Cu) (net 10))
 (segment (start 132.813 89.4) (end 133.604 88.609) (width 0.225) (layer F.Cu) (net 9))
 (segment (start 131.19 89.4) (end 132.813 89.4) (width 0.225) (layer F.Cu) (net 9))
 (segment (start 135.128 88.609) (end 133.604 88.609) (width 0.225) (layer F.Cu) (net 9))
 (segment (start 131.19 87.9) (end 131.19 86.308974) (width 0.225) (layer F.Cu) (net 11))
 (segment (start 131.19 86.308974) (end 131.808473 85.690501) (width 0.225) (layer F.Cu) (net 11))
 (segment (start 132.755001 85.690501) (end 132.817501 85.628001) (width 0.225) (layer F.Cu) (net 11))
 (segment (start 131.808473 85.690501) (end 132.755001 85.690501) (width 0.225) (layer F.Cu) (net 11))
 (segment (start 132.817501 85.628001) (end 132.817501 85.053) (width 0.225) (layer F.Cu) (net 11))
 (segment (start 132.817501 85.053) (end 133.604 85.053) (width 0.225) (layer F.Cu) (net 11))
 (segment (start 135.128 83.603) (end 135.054 83.603) (width 0.225) (layer F.Cu) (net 11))
 (segment (start 135.054 83.603) (end 133.604 85.053) (width 0.225) (layer F.Cu) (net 11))
 (segment (start 131.775136 85.053) (end 132.08 85.053) (width 0.225) (layer F.Cu) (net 7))
 (segment (start 130.54 87.25) (end 130.54 86.288136) (width 0.225) (layer F.Cu) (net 7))
 (segment (start 130.54 86.288136) (end 131.775136 85.053) (width 0.225) (layer F.Cu) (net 7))
 (segment (start 133.604 83.603) (end 133.53 83.603) (width 0.225) (layer F.Cu) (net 7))
 (segment (start 133.53 83.603) (end 132.08 85.053) (width 0.225) (layer F.Cu) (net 7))
 (segment (start 130.04 87.25) (end 130.04 85.569) (width 0.225) (layer F.Cu) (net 8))
 (segment (start 130.04 85.569) (end 130.556 85.053) (width 0.225) (layer F.Cu) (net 8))
 (segment (start 130.04 87.25) (end 130.04 85.961) (width 0.225) (layer F.Cu) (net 8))
 (segment (start 130.04 85.961) (end 129.132 85.053) (width 0.225) (layer F.Cu) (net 8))
 (segment (start 129.132 85.053) (end 129.032 85.053) (width 0.225) (layer F.Cu) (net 8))
 (segment (start 130.301 95.25) (end 130.301 97.029) (width 0.225) (layer F.Cu) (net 1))
 (segment (start 130.301 97.029) (end 129.54 97.79) (width 0.225) (layer F.Cu) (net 1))
 (segment (start 129.04 90.55) (end 129.04 90.951365) (width 0.225) (layer F.Cu) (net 1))
 (segment (start 129.04 90.951365) (end 128.771 91.220365) (width 0.225) (layer F.Cu) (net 1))
 (segment (start 128.771 91.220365) (end 128.771 93.726) (width 0.225) (layer F.Cu) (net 1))
 (segment (start 130.301 95.25) (end 129.651 95.25) (width 0.225) (layer F.Cu) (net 1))
 (segment (start 129.651 95.25) (end 128.771 94.37) (width 0.225) (layer F.Cu) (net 1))
 (segment (start 128.771 94.37) (end 128.771 93.726) (width 0.225) (layer F.Cu) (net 1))
 (segment (start 130.339 93.472) (end 129.025 93.472) (width 0.225) (layer F.Cu) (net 1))
 (segment (start 129.025 93.472) (end 128.771 93.726) (width 0.225) (layer F.Cu) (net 1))
 (segment (start 131.205001 80.884999) (end 132.08 80.01) (width 0.5) (layer F.Cu) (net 5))
 (segment (start 130.44 81.65) (end 131.205001 80.884999) (width 0.5) (layer F.Cu) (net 5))
 (segment (start 126.64699 82.74101) (end 127.798953 82.74101) (width 0.5) (layer F.Cu) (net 5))
 (segment (start 125.222 84.166) (end 126.64699 82.74101) (width 0.5) (layer F.Cu) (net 5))
 (segment (start 125.222 85.091) (end 125.222 84.166) (width 0.5) (layer F.Cu) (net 5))
 (segment (start 127.798953 82.74101) (end 128.889962 81.65) (width 0.5) (layer F.Cu) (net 5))
 (segment (start 128.889962 81.65) (end 130.44 81.65) (width 0.5) (layer F.Cu) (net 5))
 (segment (start 127.254 85.053) (end 127.154 85.053) (width 0.225) (layer F.Cu) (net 5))
 (segment (start 127.154 85.053) (end 125.702 86.505) (width 0.225) (layer F.Cu) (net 5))
 (segment (start 125.702 86.505) (end 125.476 86.505) (width 0.225) (layer F.Cu) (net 5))
 (segment (start 125.222 85.091) (end 125.222 86.251) (width 0.225) (layer F.Cu) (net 5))
 (segment (start 125.222 86.251) (end 125.476 86.505) (width 0.225) (layer F.Cu) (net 5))
 (segment (start 129.04 87.25) (end 129.04 86.625) (width 0.225) (layer F.Cu) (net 5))
 (segment (start 129.04 86.625) (end 128.92 86.505) (width 0.225) (layer F.Cu) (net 5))
 (segment (start 128.92 86.505) (end 126.751 86.505) (width 0.225) (layer F.Cu) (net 5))
 (segment (start 126.751 86.505) (end 125.476 86.505) (width 0.225) (layer F.Cu) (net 5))
 (via (at 125.1 79.7) (size 0.6858) (drill 0.3302) (layers F.Cu B.Cu) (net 2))
 (via (at 124.75 90.5) (size 0.6858) (drill 0.3302) (layers F.Cu B.Cu) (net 2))
 (via (at 125.9 97.6) (size 0.6858) (drill 0.3302) (layers F.Cu B.Cu) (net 2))
 (via (at 131.3 82.7) (size 0.6858) (drill 0.3302) (layers F.Cu B.Cu) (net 2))
 (via (at 134.392885 86.393047) (size 0.6858) (drill 0.3302) (layers F.Cu B.Cu) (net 2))
 (via (at 126.617329 90.515594) (size 0.6858) (drill 0.3302) (layers F.Cu B.Cu) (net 4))
 (via (at 129.504189 91.4747) (size 0.6858) (drill 0.3302) (layers F.Cu B.Cu) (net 4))
 (via (at 132.344301 90.063301) (size 0.6858) (drill 0.3302) (layers F.Cu B.Cu) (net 4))
 (via (at 129.035615 82.625705) (size 0.6858) (drill 0.3302) (layers F.Cu B.Cu) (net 10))
 (via (at 132.699324 87.092437) (size 0.6858) (drill 0.3302) (layers F.Cu B.Cu) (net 10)))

